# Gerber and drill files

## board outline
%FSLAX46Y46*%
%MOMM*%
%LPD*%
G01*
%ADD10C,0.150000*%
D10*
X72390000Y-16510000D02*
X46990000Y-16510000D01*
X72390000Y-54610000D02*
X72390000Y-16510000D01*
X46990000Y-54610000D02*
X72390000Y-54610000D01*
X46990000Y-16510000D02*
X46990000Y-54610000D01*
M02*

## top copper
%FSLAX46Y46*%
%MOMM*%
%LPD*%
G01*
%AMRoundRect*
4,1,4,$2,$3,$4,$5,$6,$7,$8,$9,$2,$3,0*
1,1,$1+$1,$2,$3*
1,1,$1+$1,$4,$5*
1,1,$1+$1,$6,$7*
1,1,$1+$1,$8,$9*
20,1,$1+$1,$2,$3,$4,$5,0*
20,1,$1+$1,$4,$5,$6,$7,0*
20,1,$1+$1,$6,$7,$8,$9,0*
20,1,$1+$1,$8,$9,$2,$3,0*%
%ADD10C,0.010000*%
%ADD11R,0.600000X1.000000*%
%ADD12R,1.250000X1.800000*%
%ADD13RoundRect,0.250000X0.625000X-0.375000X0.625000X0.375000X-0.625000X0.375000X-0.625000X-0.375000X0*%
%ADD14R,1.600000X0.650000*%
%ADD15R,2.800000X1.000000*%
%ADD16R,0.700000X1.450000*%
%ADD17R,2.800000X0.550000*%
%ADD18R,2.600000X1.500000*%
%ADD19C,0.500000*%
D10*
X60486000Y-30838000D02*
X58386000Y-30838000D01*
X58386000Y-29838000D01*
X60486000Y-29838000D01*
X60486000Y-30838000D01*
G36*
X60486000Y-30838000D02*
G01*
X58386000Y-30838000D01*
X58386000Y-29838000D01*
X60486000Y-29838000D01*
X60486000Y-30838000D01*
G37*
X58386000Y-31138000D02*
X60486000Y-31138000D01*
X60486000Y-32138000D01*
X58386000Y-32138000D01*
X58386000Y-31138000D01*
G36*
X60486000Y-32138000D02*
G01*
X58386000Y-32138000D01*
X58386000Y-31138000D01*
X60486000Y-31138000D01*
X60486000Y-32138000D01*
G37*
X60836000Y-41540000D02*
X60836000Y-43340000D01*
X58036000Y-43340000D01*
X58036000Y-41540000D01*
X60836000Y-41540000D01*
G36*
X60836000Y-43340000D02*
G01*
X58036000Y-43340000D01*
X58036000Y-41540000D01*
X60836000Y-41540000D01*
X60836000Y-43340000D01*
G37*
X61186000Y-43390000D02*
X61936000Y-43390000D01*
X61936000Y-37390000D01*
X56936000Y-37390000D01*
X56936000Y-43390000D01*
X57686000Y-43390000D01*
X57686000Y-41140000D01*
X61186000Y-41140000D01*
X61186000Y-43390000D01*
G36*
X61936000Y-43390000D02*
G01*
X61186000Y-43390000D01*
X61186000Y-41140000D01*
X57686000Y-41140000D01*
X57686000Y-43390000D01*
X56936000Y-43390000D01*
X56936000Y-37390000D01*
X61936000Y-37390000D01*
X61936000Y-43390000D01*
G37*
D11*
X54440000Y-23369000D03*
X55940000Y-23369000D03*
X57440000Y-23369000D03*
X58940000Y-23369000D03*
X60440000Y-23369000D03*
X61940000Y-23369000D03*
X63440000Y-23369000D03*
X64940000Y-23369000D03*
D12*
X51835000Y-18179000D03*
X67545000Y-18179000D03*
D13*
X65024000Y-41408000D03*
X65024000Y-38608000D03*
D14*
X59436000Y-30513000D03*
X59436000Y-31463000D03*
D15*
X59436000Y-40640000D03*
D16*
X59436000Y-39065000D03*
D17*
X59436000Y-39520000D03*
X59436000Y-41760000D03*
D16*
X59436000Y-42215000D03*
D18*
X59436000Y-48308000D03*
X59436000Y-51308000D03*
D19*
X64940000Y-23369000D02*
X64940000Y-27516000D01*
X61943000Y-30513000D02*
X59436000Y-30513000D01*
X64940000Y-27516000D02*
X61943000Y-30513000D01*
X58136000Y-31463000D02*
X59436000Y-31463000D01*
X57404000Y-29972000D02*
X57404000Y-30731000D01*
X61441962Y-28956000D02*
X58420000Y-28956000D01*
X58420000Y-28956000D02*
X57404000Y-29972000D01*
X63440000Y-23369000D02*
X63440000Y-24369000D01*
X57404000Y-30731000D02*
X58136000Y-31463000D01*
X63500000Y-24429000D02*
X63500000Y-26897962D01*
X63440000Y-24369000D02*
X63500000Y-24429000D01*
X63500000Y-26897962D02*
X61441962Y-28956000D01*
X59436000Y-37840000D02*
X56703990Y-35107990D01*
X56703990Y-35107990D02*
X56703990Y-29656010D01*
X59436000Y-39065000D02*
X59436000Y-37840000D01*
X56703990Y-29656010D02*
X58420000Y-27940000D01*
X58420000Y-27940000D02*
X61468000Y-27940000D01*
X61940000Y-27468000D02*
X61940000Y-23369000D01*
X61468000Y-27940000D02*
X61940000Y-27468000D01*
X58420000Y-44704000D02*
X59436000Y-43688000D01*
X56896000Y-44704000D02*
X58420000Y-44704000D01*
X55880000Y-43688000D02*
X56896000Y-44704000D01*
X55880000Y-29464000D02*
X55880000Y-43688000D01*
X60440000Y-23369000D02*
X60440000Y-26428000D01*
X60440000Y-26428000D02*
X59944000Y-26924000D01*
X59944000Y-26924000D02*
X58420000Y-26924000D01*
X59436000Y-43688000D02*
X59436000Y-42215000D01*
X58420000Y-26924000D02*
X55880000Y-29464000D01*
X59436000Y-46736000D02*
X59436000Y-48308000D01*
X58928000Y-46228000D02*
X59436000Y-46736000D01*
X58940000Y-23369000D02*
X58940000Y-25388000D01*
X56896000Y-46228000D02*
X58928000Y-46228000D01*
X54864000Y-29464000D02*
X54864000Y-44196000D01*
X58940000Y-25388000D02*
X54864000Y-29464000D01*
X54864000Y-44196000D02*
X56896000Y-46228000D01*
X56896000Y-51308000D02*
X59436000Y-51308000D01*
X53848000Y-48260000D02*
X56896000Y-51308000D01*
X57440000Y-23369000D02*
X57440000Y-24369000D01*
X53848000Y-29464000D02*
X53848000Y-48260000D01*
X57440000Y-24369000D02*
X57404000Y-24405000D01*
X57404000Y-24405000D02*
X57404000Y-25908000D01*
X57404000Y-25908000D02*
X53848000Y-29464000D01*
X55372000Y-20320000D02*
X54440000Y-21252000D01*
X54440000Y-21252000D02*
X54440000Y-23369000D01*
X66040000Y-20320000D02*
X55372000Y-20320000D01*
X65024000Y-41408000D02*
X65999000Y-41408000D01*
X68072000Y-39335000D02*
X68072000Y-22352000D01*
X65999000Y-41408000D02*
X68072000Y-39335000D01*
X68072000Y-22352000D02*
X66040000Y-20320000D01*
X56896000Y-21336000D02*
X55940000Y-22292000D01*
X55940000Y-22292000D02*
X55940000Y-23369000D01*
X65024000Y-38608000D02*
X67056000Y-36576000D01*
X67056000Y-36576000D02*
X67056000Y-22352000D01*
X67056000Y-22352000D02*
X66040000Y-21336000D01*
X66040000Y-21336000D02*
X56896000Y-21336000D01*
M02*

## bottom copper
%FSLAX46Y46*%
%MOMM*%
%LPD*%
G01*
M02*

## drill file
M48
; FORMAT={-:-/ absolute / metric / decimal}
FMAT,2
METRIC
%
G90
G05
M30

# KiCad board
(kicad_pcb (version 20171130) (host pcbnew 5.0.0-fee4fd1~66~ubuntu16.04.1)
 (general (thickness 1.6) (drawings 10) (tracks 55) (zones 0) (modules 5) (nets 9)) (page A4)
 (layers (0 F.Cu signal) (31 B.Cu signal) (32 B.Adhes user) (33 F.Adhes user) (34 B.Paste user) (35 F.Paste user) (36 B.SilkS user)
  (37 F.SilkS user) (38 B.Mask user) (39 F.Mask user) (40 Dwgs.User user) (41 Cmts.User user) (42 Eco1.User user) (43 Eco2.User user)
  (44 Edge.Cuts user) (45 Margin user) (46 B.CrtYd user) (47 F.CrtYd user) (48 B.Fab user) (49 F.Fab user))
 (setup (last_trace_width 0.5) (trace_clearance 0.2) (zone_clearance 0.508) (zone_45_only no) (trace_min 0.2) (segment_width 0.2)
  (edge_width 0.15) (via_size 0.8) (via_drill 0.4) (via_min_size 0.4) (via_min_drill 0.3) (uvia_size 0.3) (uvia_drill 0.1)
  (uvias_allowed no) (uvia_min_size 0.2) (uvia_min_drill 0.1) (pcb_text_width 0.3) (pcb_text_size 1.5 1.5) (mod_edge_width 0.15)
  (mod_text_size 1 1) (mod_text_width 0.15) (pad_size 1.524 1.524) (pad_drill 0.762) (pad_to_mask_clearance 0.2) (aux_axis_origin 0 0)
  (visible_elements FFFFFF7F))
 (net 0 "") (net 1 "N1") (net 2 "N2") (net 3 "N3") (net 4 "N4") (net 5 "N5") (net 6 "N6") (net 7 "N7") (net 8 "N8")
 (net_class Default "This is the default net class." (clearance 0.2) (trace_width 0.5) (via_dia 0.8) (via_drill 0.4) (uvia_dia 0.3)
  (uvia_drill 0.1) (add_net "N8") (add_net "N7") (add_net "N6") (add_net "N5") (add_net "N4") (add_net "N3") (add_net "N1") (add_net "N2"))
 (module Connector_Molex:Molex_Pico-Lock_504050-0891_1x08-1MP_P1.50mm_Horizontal (layer F.Cu) (at 59.69 20.574)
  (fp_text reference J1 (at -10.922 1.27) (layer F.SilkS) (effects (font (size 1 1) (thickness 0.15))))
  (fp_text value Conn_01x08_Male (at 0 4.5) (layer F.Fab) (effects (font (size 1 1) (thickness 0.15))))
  (pad 1 smd rect (at -5.25 2.795) (size 0.6 1) (layers F.Cu F.Paste F.Mask) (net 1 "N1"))
  (pad 2 smd rect (at -3.75 2.795) (size 0.6 1) (layers F.Cu F.Paste F.Mask) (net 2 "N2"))
  (pad 3 smd rect (at -2.25 2.795) (size 0.6 1) (layers F.Cu F.Paste F.Mask) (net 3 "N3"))
  (pad 4 smd rect (at -0.75 2.795) (size 0.6 1) (layers F.Cu F.Paste F.Mask) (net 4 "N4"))
  (pad 5 smd rect (at 0.75 2.795) (size 0.6 1) (layers F.Cu F.Paste F.Mask) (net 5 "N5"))
  (pad 6 smd rect (at 2.25 2.795) (size 0.6 1) (layers F.Cu F.Paste F.Mask) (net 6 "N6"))
  (pad 7 smd rect (at 3.75 2.795) (size 0.6 1) (layers F.Cu F.Paste F.Mask) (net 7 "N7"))
  (pad 8 smd rect (at 5.25 2.795) (size 0.6 1) (layers F.Cu F.Paste F.Mask) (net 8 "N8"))
  (pad MP smd rect (at -7.855 -2.395) (size 1.25 1.8) (layers F.Cu F.Paste F.Mask))
  (pad MP smd rect (at 7.855 -2.395) (size 1.25 1.8) (layers F.Cu F.Paste F.Mask)))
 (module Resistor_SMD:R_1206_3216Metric (layer F.Cu) (at 65.024 40.008 90)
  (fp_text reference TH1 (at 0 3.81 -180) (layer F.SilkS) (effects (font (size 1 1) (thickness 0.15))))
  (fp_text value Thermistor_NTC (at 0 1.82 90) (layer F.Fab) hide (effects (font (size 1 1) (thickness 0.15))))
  (pad 1 smd roundrect (at -1.4 0 90) (size 1.25 1.75) (layers F.Cu F.Paste F.Mask) (roundrect_rratio 0.2) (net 1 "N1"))
  (pad 2 smd roundrect (at 1.4 0 90) (size 1.25 1.75) (layers F.Cu F.Paste F.Mask) (roundrect_rratio 0.2) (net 2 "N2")))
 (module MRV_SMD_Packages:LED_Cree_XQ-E (layer F.Cu) (at 59.436 30.988 270)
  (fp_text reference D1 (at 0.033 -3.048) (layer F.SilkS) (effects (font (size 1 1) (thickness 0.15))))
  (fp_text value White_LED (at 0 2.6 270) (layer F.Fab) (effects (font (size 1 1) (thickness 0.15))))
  (fp_poly (pts (xy -0.15 -1.05) (xy -0.15 1.05) (xy -1.15 1.05) (xy -1.15 -1.05)) (layer F.Cu) (width 0.01))
  (fp_poly (pts (xy 0.15 1.05) (xy 0.15 -1.05) (xy 1.15 -1.05) (xy 1.15 1.05)) (layer F.Cu) (width 0.01))
  (pad 1 smd rect (at -0.475 0 270) (size 0.65 1.6) (layers F.Cu F.Paste F.Mask) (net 8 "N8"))
  (pad 2 smd rect (at 0.475 0 90) (size 0.65 1.6) (layers F.Cu F.Paste F.Mask) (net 7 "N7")))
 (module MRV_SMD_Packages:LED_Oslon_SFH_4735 (layer F.Cu) (at 59.436 40.64 180)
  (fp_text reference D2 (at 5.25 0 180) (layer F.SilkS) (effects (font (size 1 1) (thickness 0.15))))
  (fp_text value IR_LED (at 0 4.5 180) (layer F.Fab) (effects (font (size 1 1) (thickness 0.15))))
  (fp_poly (pts (xy -1.4 -0.9) (xy -1.4 -2.7) (xy 1.4 -2.7) (xy 1.4 -0.9)) (layer F.Cu) (width 0.01))
  (fp_poly
   (pts (xy -1.75 -2.75) (xy -2.5 -2.75) (xy -2.5 3.25) (xy 2.5 3.25) (xy 2.5 -2.75) (xy 1.75 -2.75) (xy 1.75 -0.5) (xy -1.75 -0.5))
   (layer F.Cu) (width 0.01))
  (pad 1 smd rect (at 0 0 180) (size 2.8 1) (layers F.Cu F.Paste F.Mask) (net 6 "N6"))
  (pad 1 smd rect (at 0 1.575 180) (size 0.7 1.45) (layers F.Cu F.Paste F.Mask) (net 6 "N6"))
  (pad 1 smd rect (at 0 1.12 180) (size 2.8 0.55) (layers F.Cu F.Paste F.Mask) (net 6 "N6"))
  (pad 2 smd rect (at 0 -1.12) (size 2.8 0.55) (layers F.Cu F.Paste F.Mask) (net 5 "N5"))
  (pad 2 smd rect (at 0 -1.575) (size 0.7 1.45) (layers F.Cu F.Paste F.Mask) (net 5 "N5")))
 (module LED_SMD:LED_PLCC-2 (layer F.Cu) (at 59.436 49.808 270)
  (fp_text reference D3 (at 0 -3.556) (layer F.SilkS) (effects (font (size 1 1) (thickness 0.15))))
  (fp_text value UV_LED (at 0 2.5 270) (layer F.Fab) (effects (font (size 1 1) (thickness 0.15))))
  (pad 1 smd rect (at -1.5 0 270) (size 1.5 2.6) (layers F.Cu F.Paste F.Mask) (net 4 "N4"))
  (pad 2 smd rect (at 1.5 0 270) (size 1.5 2.6) (layers F.Cu F.Paste F.Mask) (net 3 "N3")))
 (gr_line (start 72.39 16.51) (end 46.99 16.51) (layer Edge.Cuts) (width 0.15))
 (gr_line (start 72.39 54.61) (end 72.39 16.51) (layer Edge.Cuts) (width 0.15))
 (gr_line (start 46.99 54.61) (end 72.39 54.61) (layer Edge.Cuts) (width 0.15))
 (gr_line (start 46.99 16.51) (end 46.99 54.61) (layer Edge.Cuts) (width 0.15))
 (segment (start 64.94 23.369) (end 64.94 27.516) (width 0.5) (layer F.Cu) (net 8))
 (segment (start 61.943 30.513) (end 59.436 30.513) (width 0.5) (layer F.Cu) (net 8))
 (segment (start 64.94 27.516) (end 61.943 30.513) (width 0.5) (layer F.Cu) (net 8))
 (segment (start 58.136 31.463) (end 59.436 31.463) (width 0.5) (layer F.Cu) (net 7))
 (segment (start 57.404 29.972) (end 57.404 30.731) (width 0.5) (layer F.Cu) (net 7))
 (segment (start 61.441962 28.956) (end 58.42 28.956) (width 0.5) (layer F.Cu) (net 7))
 (segment (start 58.42 28.956) (end 57.404 29.972) (width 0.5) (layer F.Cu) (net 7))
 (segment (start 63.44 23.369) (end 63.44 24.369) (width 0.5) (layer F.Cu) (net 7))
 (segment (start 57.404 30.731) (end 58.136 31.463) (width 0.5) (layer F.Cu) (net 7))
 (segment (start 63.5 24.429) (end 63.5 26.897962) (width 0.5) (layer F.Cu) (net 7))
 (segment (start 63.44 24.369) (end 63.5 24.429) (width 0.5) (layer F.Cu) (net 7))
 (segment (start 63.5 26.897962) (end 61.441962 28.956) (width 0.5) (layer F.Cu) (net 7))
 (segment (start 59.436 37.84) (end 56.70399 35.10799) (width 0.5) (layer F.Cu) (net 6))
 (segment (start 56.70399 35.10799) (end 56.70399 29.65601) (width 0.5) (layer F.Cu) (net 6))
 (segment (start 59.436 39.065) (end 59.436 37.84) (width 0.5) (layer F.Cu) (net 6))
 (segment (start 56.70399 29.65601) (end 58.42 27.94) (width 0.5) (layer F.Cu) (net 6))
 (segment (start 58.42 27.94) (end 61.468 27.94) (width 0.5) (layer F.Cu) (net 6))
 (segment (start 61.94 27.468) (end 61.94 23.369) (width 0.5) (layer F.Cu) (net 6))
 (segment (start 61.468 27.94) (end 61.94 27.468) (width 0.5) (layer F.Cu) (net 6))
 (segment (start 58.42 44.704) (end 59.436 43.688) (width 0.5) (layer F.Cu) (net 5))
 (segment (start 56.896 44.704) (end 58.42 44.704) (width 0.5) (layer F.Cu) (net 5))
 (segment (start 55.88 43.688) (end 56.896 44.704) (width 0.5) (layer F.Cu) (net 5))
 (segment (start 55.88 29.464) (end 55.88 43.688) (width 0.5) (layer F.Cu) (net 5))
 (segment (start 60.44 23.369) (end 60.44 26.428) (width 0.5) (layer F.Cu) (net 5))
 (segment (start 60.44 26.428) (end 59.944 26.924) (width 0.5) (layer F.Cu) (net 5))
 (segment (start 59.944 26.924) (end 58.42 26.924) (width 0.5) (layer F.Cu) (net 5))
 (segment (start 59.436 43.688) (end 59.436 42.215) (width 0.5) (layer F.Cu) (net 5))
 (segment (start 58.42 26.924) (end 55.88 29.464) (width 0.5) (layer F.Cu) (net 5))
 (segment (start 59.436 46.736) (end 59.436 48.308) (width 0.5) (layer F.Cu) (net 4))
 (segment (start 58.928 46.228) (end 59.436 46.736) (width 0.5) (layer F.Cu) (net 4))
 (segment (start 58.94 23.369) (end 58.94 25.388) (width 0.5) (layer F.Cu) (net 4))
 (segment (start 56.896 46.228) (end 58.928 46.228) (width 0.5) (layer F.Cu) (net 4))
 (segment (start 54.864 29.464) (end 54.864 44.196) (width 0.5) (layer F.Cu) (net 4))
 (segment (start 58.94 25.388) (end 54.864 29.464) (width 0.5) (layer F.Cu) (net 4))
 (segment (start 54.864 44.196) (end 56.896 46.228) (width 0.5) (layer F.Cu) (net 4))
 (segment (start 56.896 51.308) (end 59.436 51.308) (width 0.5) (layer F.Cu) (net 3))
 (segment (start 53.848 48.26) (end 56.896 51.308) (width 0.5) (layer F.Cu) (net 3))
 (segment (start 57.44 23.369) (end 57.44 24.369) (width 0.5) (layer F.Cu) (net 3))
 (segment (start 53.848 29.464) (end 53.848 48.26) (width 0.5) (layer F.Cu) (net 3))
 (segment (start 57.44 24.369) (end 57.404 24.405) (width 0.5) (layer F.Cu) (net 3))
 (segment (start 57.404 24.405) (end 57.404 25.908) (width 0.5) (layer F.Cu) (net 3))
 (segment (start 57.404 25.908) (end 53.848 29.464) (width 0.5) (layer F.Cu) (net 3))
 (segment (start 55.372 20.32) (end 54.44 21.252) (width 0.5) (layer F.Cu) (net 1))
 (segment (start 54.44 21.252) (end 54.44 23.369) (width 0.5) (layer F.Cu) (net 1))
 (segment (start 66.04 20.32) (end 55.372 20.32) (width 0.5) (layer F.Cu) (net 1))
 (segment (start 65.024 41.408) (end 65.999 41.408) (width 0.5) (layer F.Cu) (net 1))
 (segment (start 68.072 39.335) (end 68.072 22.352) (width 0.5) (layer F.Cu) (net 1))
 (segment (start 65.999 41.408) (end 68.072 39.335) (width 0.5) (layer F.Cu) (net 1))
 (segment (start 68.072 22.352) (end 66.04 20.32) (width 0.5) (layer F.Cu) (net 1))
 (segment (start 56.896 21.336) (end 55.94 22.292) (width 0.5) (layer F.Cu) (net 2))
 (segment (start 55.94 22.292) (end 55.94 23.369) (width 0.5) (layer F.Cu) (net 2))
 (segment (start 65.024 38.608) (end 67.056 36.576) (width 0.5) (layer F.Cu) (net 2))
 (segment (start 67.056 36.576) (end 67.056 22.352) (width 0.5) (layer F.Cu) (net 2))
 (segment (start 67.056 22.352) (end 66.04 21.336) (width 0.5) (layer F.Cu) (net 2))
 (segment (start 66.04 21.336) (end 56.896 21.336) (width 0.5) (layer F.Cu) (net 2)))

